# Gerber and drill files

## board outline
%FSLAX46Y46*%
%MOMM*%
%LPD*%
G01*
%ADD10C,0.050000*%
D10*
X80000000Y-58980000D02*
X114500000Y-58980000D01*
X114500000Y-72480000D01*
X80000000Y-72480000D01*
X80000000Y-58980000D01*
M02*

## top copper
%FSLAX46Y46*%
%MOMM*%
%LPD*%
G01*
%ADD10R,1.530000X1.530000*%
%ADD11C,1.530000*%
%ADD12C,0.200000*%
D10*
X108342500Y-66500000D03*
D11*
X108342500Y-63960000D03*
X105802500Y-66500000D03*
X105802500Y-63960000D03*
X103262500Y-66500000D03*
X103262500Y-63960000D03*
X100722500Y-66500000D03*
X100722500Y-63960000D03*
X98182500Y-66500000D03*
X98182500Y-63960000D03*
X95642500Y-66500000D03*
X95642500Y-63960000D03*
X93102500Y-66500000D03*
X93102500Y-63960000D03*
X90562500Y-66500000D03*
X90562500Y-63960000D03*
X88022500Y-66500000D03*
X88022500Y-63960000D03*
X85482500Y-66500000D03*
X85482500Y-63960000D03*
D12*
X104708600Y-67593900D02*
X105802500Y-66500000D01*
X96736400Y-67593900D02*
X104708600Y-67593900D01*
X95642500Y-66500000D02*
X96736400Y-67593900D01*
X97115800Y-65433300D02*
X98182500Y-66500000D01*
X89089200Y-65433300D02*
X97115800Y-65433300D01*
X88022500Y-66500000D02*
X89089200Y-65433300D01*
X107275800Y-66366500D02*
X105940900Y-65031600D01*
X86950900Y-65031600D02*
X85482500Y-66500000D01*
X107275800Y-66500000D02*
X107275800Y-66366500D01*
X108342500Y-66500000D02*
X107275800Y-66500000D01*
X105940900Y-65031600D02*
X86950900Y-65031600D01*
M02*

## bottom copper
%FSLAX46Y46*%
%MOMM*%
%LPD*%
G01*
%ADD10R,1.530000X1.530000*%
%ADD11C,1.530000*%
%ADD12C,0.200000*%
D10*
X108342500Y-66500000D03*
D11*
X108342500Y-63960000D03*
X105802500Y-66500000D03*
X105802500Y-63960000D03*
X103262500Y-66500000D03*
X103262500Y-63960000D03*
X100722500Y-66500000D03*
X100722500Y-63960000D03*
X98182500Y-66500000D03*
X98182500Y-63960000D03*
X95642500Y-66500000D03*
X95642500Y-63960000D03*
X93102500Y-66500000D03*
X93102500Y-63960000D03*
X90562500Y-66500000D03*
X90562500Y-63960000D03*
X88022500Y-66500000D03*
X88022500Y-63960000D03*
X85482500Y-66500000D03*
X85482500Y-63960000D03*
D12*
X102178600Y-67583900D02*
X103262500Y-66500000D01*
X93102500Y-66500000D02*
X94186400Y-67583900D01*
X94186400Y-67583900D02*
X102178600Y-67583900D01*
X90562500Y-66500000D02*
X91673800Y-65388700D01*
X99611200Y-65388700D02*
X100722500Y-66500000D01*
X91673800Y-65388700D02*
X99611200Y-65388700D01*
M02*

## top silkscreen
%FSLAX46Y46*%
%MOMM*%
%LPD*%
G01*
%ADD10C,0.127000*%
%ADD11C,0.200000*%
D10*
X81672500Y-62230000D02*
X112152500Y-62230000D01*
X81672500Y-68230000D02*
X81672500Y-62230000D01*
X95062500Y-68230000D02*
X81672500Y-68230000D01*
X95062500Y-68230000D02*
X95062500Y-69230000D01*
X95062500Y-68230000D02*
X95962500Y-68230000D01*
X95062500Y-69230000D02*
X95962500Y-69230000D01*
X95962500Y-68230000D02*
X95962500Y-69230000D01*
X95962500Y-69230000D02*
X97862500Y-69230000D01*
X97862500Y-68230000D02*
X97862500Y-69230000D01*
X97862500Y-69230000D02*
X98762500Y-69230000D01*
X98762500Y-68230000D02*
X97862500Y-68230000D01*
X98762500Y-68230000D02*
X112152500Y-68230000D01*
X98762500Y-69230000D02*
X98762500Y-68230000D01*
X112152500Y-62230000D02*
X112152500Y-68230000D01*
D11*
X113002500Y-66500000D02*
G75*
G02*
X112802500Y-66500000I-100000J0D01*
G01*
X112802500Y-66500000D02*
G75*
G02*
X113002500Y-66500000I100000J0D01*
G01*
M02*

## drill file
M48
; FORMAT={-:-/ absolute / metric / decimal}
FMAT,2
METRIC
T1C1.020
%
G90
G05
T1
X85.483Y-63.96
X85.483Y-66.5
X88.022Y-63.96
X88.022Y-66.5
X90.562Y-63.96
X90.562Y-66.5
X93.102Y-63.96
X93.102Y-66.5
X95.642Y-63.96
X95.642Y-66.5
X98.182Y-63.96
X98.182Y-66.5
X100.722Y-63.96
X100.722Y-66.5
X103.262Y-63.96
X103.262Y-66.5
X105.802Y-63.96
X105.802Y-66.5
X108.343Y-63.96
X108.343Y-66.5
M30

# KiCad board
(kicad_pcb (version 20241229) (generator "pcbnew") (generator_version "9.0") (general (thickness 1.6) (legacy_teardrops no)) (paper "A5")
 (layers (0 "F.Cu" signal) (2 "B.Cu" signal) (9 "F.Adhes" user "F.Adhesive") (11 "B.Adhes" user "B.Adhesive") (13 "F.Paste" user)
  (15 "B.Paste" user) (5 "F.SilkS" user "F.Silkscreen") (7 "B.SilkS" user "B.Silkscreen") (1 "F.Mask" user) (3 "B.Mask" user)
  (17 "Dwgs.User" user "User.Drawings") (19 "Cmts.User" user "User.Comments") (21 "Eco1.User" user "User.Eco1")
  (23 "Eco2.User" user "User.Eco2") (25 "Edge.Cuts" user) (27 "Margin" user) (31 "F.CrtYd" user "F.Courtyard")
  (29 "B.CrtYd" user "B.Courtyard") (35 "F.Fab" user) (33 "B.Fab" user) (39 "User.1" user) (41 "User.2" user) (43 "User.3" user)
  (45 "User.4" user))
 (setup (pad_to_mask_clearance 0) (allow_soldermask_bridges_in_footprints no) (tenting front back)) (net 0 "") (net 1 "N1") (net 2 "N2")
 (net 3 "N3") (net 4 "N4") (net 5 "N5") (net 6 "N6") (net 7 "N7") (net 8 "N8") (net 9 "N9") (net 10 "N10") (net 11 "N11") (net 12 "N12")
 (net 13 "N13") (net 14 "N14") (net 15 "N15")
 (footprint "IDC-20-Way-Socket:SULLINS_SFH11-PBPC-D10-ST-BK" (layer "F.Cu") (at 96.9125 65.23)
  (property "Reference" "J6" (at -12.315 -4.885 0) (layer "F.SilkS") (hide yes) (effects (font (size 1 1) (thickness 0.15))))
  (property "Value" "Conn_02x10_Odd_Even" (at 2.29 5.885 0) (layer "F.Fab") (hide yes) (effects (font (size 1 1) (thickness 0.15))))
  (fp_line (start -15.24 -3) (end 15.24 -3) (stroke (width 0.127) (type solid)) (layer "F.SilkS"))
  (fp_line (start -15.24 3) (end -15.24 -3) (stroke (width 0.127) (type solid)) (layer "F.SilkS"))
  (fp_line (start -1.85 3) (end -15.24 3) (stroke (width 0.127) (type solid)) (layer "F.SilkS"))
  (fp_line (start -1.85 3) (end -1.85 4) (stroke (width 0.127) (type solid)) (layer "F.SilkS"))
  (fp_line (start -1.85 3) (end -0.95 3) (stroke (width 0.127) (type solid)) (layer "F.SilkS"))
  (fp_line (start -1.85 4) (end -0.95 4) (stroke (width 0.127) (type solid)) (layer "F.SilkS"))
  (fp_line (start -0.95 3) (end -0.95 4) (stroke (width 0.127) (type solid)) (layer "F.SilkS"))
  (fp_line (start -0.95 4) (end 0.95 4) (stroke (width 0.127) (type solid)) (layer "F.SilkS"))
  (fp_line (start 0.95 3) (end 0.95 4) (stroke (width 0.127) (type solid)) (layer "F.SilkS"))
  (fp_line (start 0.95 4) (end 1.85 4) (stroke (width 0.127) (type solid)) (layer "F.SilkS"))
  (fp_line (start 1.85 3) (end 0.95 3) (stroke (width 0.127) (type solid)) (layer "F.SilkS"))
  (fp_line (start 1.85 3) (end 15.24 3) (stroke (width 0.127) (type solid)) (layer "F.SilkS"))
  (fp_line (start 1.85 4) (end 1.85 3) (stroke (width 0.127) (type solid)) (layer "F.SilkS"))
  (fp_line (start 15.24 -3) (end 15.24 3) (stroke (width 0.127) (type solid)) (layer "F.SilkS"))
  (fp_circle (center 15.99 1.27) (end 16.09 1.27) (stroke (width 0.2) (type solid)) (fill no) (layer "F.SilkS"))
  (pad "1" thru_hole rect (at 11.43 1.27) (size 1.53 1.53) (drill 1.02) (layers "*.Cu" "*.Mask") (remove_unused_layers no) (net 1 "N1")
   (solder_mask_margin 0.102))
  (pad "2" thru_hole circle (at 11.43 -1.27) (size 1.53 1.53) (drill 1.02) (layers "*.Cu" "*.Mask") (remove_unused_layers no) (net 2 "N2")
   (solder_mask_margin 0.102))
  (pad "3" thru_hole circle (at 8.89 1.27) (size 1.53 1.53) (drill 1.02) (layers "*.Cu" "*.Mask") (remove_unused_layers no) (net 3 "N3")
   (solder_mask_margin 0.102))
  (pad "4" thru_hole circle (at 8.89 -1.27) (size 1.53 1.53) (drill 1.02) (layers "*.Cu" "*.Mask") (remove_unused_layers no) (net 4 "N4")
   (solder_mask_margin 0.102))
  (pad "5" thru_hole circle (at 6.35 1.27) (size 1.53 1.53) (drill 1.02) (layers "*.Cu" "*.Mask") (remove_unused_layers no) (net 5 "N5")
   (solder_mask_margin 0.102))
  (pad "6" thru_hole circle (at 6.35 -1.27) (size 1.53 1.53) (drill 1.02) (layers "*.Cu" "*.Mask") (remove_unused_layers no) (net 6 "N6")
   (solder_mask_margin 0.102))
  (pad "7" thru_hole circle (at 3.81 1.27) (size 1.53 1.53) (drill 1.02) (layers "*.Cu" "*.Mask") (remove_unused_layers no) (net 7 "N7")
   (solder_mask_margin 0.102))
  (pad "8" thru_hole circle (at 3.81 -1.27) (size 1.53 1.53) (drill 1.02) (layers "*.Cu" "*.Mask") (remove_unused_layers no) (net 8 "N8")
   (solder_mask_margin 0.102))
  (pad "9" thru_hole circle (at 1.27 1.27) (size 1.53 1.53) (drill 1.02) (layers "*.Cu" "*.Mask") (remove_unused_layers no) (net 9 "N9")
   (solder_mask_margin 0.102))
  (pad "10" thru_hole circle (at 1.27 -1.27) (size 1.53 1.53) (drill 1.02) (layers "*.Cu" "*.Mask") (remove_unused_layers no) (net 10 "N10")
   (solder_mask_margin 0.102))
  (pad "11" thru_hole circle (at -1.27 1.27) (size 1.53 1.53) (drill 1.02) (layers "*.Cu" "*.Mask") (remove_unused_layers no) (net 3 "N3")
   (solder_mask_margin 0.102))
  (pad "12" thru_hole circle (at -1.27 -1.27) (size 1.53 1.53) (drill 1.02) (layers "*.Cu" "*.Mask") (remove_unused_layers no)
   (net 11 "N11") (solder_mask_margin 0.102))
  (pad "13" thru_hole circle (at -3.81 1.27) (size 1.53 1.53) (drill 1.02) (layers "*.Cu" "*.Mask") (remove_unused_layers no) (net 5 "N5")
   (solder_mask_margin 0.102))
  (pad "14" thru_hole circle (at -3.81 -1.27) (size 1.53 1.53) (drill 1.02) (layers "*.Cu" "*.Mask") (remove_unused_layers no)
   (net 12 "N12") (solder_mask_margin 0.102))
  (pad "15" thru_hole circle (at -6.35 1.27) (size 1.53 1.53) (drill 1.02) (layers "*.Cu" "*.Mask") (remove_unused_layers no) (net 7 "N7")
   (solder_mask_margin 0.102))
  (pad "16" thru_hole circle (at -6.35 -1.27) (size 1.53 1.53) (drill 1.02) (layers "*.Cu" "*.Mask") (remove_unused_layers no)
   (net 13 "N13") (solder_mask_margin 0.102))
  (pad "17" thru_hole circle (at -8.89 1.27) (size 1.53 1.53) (drill 1.02) (layers "*.Cu" "*.Mask") (remove_unused_layers no) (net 9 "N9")
   (solder_mask_margin 0.102))
  (pad "18" thru_hole circle (at -8.89 -1.27) (size 1.53 1.53) (drill 1.02) (layers "*.Cu" "*.Mask") (remove_unused_layers no)
   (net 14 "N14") (solder_mask_margin 0.102))
  (pad "19" thru_hole circle (at -11.43 1.27) (size 1.53 1.53) (drill 1.02) (layers "*.Cu" "*.Mask") (remove_unused_layers no) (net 1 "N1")
   (solder_mask_margin 0.102))
  (pad "20" thru_hole circle (at -11.43 -1.27) (size 1.53 1.53) (drill 1.02) (layers "*.Cu" "*.Mask") (remove_unused_layers no)
   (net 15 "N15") (solder_mask_margin 0.102)))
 (gr_rect (start 80 58.98) (end 114.5 72.48) (stroke (width 0.05) (type default)) (fill no) (layer "Edge.Cuts"))
 (segment (start 104.7086 67.5939) (end 105.8025 66.5) (width 0.2) (layer "F.Cu") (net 3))
 (segment (start 96.7364 67.5939) (end 104.7086 67.5939) (width 0.2) (layer "F.Cu") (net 3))
 (segment (start 95.6425 66.5) (end 96.7364 67.5939) (width 0.2) (layer "F.Cu") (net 3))
 (segment (start 102.1786 67.5839) (end 103.2625 66.5) (width 0.2) (layer "B.Cu") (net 5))
 (segment (start 93.1025 66.5) (end 94.1864 67.5839) (width 0.2) (layer "B.Cu") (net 5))
 (segment (start 94.1864 67.5839) (end 102.1786 67.5839) (width 0.2) (layer "B.Cu") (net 5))
 (segment (start 97.1158 65.4333) (end 98.1825 66.5) (width 0.2) (layer "F.Cu") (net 9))
 (segment (start 89.0892 65.4333) (end 97.1158 65.4333) (width 0.2) (layer "F.Cu") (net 9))
 (segment (start 88.0225 66.5) (end 89.0892 65.4333) (width 0.2) (layer "F.Cu") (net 9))
 (segment (start 107.2758 66.3665) (end 105.9409 65.0316) (width 0.2) (layer "F.Cu") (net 1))
 (segment (start 86.9509 65.0316) (end 85.4825 66.5) (width 0.2) (layer "F.Cu") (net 1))
 (segment (start 107.2758 66.5) (end 107.2758 66.3665) (width 0.2) (layer "F.Cu") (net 1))
 (segment (start 108.3425 66.5) (end 107.2758 66.5) (width 0.2) (layer "F.Cu") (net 1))
 (segment (start 105.9409 65.0316) (end 86.9509 65.0316) (width 0.2) (layer "F.Cu") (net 1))
 (segment (start 90.5625 66.5) (end 91.6738 65.3887) (width 0.2) (layer "B.Cu") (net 7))
 (segment (start 99.6112 65.3887) (end 100.7225 66.5) (width 0.2) (layer "B.Cu") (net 7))
 (segment (start 91.6738 65.3887) (end 99.6112 65.3887) (width 0.2) (layer "B.Cu") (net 7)))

